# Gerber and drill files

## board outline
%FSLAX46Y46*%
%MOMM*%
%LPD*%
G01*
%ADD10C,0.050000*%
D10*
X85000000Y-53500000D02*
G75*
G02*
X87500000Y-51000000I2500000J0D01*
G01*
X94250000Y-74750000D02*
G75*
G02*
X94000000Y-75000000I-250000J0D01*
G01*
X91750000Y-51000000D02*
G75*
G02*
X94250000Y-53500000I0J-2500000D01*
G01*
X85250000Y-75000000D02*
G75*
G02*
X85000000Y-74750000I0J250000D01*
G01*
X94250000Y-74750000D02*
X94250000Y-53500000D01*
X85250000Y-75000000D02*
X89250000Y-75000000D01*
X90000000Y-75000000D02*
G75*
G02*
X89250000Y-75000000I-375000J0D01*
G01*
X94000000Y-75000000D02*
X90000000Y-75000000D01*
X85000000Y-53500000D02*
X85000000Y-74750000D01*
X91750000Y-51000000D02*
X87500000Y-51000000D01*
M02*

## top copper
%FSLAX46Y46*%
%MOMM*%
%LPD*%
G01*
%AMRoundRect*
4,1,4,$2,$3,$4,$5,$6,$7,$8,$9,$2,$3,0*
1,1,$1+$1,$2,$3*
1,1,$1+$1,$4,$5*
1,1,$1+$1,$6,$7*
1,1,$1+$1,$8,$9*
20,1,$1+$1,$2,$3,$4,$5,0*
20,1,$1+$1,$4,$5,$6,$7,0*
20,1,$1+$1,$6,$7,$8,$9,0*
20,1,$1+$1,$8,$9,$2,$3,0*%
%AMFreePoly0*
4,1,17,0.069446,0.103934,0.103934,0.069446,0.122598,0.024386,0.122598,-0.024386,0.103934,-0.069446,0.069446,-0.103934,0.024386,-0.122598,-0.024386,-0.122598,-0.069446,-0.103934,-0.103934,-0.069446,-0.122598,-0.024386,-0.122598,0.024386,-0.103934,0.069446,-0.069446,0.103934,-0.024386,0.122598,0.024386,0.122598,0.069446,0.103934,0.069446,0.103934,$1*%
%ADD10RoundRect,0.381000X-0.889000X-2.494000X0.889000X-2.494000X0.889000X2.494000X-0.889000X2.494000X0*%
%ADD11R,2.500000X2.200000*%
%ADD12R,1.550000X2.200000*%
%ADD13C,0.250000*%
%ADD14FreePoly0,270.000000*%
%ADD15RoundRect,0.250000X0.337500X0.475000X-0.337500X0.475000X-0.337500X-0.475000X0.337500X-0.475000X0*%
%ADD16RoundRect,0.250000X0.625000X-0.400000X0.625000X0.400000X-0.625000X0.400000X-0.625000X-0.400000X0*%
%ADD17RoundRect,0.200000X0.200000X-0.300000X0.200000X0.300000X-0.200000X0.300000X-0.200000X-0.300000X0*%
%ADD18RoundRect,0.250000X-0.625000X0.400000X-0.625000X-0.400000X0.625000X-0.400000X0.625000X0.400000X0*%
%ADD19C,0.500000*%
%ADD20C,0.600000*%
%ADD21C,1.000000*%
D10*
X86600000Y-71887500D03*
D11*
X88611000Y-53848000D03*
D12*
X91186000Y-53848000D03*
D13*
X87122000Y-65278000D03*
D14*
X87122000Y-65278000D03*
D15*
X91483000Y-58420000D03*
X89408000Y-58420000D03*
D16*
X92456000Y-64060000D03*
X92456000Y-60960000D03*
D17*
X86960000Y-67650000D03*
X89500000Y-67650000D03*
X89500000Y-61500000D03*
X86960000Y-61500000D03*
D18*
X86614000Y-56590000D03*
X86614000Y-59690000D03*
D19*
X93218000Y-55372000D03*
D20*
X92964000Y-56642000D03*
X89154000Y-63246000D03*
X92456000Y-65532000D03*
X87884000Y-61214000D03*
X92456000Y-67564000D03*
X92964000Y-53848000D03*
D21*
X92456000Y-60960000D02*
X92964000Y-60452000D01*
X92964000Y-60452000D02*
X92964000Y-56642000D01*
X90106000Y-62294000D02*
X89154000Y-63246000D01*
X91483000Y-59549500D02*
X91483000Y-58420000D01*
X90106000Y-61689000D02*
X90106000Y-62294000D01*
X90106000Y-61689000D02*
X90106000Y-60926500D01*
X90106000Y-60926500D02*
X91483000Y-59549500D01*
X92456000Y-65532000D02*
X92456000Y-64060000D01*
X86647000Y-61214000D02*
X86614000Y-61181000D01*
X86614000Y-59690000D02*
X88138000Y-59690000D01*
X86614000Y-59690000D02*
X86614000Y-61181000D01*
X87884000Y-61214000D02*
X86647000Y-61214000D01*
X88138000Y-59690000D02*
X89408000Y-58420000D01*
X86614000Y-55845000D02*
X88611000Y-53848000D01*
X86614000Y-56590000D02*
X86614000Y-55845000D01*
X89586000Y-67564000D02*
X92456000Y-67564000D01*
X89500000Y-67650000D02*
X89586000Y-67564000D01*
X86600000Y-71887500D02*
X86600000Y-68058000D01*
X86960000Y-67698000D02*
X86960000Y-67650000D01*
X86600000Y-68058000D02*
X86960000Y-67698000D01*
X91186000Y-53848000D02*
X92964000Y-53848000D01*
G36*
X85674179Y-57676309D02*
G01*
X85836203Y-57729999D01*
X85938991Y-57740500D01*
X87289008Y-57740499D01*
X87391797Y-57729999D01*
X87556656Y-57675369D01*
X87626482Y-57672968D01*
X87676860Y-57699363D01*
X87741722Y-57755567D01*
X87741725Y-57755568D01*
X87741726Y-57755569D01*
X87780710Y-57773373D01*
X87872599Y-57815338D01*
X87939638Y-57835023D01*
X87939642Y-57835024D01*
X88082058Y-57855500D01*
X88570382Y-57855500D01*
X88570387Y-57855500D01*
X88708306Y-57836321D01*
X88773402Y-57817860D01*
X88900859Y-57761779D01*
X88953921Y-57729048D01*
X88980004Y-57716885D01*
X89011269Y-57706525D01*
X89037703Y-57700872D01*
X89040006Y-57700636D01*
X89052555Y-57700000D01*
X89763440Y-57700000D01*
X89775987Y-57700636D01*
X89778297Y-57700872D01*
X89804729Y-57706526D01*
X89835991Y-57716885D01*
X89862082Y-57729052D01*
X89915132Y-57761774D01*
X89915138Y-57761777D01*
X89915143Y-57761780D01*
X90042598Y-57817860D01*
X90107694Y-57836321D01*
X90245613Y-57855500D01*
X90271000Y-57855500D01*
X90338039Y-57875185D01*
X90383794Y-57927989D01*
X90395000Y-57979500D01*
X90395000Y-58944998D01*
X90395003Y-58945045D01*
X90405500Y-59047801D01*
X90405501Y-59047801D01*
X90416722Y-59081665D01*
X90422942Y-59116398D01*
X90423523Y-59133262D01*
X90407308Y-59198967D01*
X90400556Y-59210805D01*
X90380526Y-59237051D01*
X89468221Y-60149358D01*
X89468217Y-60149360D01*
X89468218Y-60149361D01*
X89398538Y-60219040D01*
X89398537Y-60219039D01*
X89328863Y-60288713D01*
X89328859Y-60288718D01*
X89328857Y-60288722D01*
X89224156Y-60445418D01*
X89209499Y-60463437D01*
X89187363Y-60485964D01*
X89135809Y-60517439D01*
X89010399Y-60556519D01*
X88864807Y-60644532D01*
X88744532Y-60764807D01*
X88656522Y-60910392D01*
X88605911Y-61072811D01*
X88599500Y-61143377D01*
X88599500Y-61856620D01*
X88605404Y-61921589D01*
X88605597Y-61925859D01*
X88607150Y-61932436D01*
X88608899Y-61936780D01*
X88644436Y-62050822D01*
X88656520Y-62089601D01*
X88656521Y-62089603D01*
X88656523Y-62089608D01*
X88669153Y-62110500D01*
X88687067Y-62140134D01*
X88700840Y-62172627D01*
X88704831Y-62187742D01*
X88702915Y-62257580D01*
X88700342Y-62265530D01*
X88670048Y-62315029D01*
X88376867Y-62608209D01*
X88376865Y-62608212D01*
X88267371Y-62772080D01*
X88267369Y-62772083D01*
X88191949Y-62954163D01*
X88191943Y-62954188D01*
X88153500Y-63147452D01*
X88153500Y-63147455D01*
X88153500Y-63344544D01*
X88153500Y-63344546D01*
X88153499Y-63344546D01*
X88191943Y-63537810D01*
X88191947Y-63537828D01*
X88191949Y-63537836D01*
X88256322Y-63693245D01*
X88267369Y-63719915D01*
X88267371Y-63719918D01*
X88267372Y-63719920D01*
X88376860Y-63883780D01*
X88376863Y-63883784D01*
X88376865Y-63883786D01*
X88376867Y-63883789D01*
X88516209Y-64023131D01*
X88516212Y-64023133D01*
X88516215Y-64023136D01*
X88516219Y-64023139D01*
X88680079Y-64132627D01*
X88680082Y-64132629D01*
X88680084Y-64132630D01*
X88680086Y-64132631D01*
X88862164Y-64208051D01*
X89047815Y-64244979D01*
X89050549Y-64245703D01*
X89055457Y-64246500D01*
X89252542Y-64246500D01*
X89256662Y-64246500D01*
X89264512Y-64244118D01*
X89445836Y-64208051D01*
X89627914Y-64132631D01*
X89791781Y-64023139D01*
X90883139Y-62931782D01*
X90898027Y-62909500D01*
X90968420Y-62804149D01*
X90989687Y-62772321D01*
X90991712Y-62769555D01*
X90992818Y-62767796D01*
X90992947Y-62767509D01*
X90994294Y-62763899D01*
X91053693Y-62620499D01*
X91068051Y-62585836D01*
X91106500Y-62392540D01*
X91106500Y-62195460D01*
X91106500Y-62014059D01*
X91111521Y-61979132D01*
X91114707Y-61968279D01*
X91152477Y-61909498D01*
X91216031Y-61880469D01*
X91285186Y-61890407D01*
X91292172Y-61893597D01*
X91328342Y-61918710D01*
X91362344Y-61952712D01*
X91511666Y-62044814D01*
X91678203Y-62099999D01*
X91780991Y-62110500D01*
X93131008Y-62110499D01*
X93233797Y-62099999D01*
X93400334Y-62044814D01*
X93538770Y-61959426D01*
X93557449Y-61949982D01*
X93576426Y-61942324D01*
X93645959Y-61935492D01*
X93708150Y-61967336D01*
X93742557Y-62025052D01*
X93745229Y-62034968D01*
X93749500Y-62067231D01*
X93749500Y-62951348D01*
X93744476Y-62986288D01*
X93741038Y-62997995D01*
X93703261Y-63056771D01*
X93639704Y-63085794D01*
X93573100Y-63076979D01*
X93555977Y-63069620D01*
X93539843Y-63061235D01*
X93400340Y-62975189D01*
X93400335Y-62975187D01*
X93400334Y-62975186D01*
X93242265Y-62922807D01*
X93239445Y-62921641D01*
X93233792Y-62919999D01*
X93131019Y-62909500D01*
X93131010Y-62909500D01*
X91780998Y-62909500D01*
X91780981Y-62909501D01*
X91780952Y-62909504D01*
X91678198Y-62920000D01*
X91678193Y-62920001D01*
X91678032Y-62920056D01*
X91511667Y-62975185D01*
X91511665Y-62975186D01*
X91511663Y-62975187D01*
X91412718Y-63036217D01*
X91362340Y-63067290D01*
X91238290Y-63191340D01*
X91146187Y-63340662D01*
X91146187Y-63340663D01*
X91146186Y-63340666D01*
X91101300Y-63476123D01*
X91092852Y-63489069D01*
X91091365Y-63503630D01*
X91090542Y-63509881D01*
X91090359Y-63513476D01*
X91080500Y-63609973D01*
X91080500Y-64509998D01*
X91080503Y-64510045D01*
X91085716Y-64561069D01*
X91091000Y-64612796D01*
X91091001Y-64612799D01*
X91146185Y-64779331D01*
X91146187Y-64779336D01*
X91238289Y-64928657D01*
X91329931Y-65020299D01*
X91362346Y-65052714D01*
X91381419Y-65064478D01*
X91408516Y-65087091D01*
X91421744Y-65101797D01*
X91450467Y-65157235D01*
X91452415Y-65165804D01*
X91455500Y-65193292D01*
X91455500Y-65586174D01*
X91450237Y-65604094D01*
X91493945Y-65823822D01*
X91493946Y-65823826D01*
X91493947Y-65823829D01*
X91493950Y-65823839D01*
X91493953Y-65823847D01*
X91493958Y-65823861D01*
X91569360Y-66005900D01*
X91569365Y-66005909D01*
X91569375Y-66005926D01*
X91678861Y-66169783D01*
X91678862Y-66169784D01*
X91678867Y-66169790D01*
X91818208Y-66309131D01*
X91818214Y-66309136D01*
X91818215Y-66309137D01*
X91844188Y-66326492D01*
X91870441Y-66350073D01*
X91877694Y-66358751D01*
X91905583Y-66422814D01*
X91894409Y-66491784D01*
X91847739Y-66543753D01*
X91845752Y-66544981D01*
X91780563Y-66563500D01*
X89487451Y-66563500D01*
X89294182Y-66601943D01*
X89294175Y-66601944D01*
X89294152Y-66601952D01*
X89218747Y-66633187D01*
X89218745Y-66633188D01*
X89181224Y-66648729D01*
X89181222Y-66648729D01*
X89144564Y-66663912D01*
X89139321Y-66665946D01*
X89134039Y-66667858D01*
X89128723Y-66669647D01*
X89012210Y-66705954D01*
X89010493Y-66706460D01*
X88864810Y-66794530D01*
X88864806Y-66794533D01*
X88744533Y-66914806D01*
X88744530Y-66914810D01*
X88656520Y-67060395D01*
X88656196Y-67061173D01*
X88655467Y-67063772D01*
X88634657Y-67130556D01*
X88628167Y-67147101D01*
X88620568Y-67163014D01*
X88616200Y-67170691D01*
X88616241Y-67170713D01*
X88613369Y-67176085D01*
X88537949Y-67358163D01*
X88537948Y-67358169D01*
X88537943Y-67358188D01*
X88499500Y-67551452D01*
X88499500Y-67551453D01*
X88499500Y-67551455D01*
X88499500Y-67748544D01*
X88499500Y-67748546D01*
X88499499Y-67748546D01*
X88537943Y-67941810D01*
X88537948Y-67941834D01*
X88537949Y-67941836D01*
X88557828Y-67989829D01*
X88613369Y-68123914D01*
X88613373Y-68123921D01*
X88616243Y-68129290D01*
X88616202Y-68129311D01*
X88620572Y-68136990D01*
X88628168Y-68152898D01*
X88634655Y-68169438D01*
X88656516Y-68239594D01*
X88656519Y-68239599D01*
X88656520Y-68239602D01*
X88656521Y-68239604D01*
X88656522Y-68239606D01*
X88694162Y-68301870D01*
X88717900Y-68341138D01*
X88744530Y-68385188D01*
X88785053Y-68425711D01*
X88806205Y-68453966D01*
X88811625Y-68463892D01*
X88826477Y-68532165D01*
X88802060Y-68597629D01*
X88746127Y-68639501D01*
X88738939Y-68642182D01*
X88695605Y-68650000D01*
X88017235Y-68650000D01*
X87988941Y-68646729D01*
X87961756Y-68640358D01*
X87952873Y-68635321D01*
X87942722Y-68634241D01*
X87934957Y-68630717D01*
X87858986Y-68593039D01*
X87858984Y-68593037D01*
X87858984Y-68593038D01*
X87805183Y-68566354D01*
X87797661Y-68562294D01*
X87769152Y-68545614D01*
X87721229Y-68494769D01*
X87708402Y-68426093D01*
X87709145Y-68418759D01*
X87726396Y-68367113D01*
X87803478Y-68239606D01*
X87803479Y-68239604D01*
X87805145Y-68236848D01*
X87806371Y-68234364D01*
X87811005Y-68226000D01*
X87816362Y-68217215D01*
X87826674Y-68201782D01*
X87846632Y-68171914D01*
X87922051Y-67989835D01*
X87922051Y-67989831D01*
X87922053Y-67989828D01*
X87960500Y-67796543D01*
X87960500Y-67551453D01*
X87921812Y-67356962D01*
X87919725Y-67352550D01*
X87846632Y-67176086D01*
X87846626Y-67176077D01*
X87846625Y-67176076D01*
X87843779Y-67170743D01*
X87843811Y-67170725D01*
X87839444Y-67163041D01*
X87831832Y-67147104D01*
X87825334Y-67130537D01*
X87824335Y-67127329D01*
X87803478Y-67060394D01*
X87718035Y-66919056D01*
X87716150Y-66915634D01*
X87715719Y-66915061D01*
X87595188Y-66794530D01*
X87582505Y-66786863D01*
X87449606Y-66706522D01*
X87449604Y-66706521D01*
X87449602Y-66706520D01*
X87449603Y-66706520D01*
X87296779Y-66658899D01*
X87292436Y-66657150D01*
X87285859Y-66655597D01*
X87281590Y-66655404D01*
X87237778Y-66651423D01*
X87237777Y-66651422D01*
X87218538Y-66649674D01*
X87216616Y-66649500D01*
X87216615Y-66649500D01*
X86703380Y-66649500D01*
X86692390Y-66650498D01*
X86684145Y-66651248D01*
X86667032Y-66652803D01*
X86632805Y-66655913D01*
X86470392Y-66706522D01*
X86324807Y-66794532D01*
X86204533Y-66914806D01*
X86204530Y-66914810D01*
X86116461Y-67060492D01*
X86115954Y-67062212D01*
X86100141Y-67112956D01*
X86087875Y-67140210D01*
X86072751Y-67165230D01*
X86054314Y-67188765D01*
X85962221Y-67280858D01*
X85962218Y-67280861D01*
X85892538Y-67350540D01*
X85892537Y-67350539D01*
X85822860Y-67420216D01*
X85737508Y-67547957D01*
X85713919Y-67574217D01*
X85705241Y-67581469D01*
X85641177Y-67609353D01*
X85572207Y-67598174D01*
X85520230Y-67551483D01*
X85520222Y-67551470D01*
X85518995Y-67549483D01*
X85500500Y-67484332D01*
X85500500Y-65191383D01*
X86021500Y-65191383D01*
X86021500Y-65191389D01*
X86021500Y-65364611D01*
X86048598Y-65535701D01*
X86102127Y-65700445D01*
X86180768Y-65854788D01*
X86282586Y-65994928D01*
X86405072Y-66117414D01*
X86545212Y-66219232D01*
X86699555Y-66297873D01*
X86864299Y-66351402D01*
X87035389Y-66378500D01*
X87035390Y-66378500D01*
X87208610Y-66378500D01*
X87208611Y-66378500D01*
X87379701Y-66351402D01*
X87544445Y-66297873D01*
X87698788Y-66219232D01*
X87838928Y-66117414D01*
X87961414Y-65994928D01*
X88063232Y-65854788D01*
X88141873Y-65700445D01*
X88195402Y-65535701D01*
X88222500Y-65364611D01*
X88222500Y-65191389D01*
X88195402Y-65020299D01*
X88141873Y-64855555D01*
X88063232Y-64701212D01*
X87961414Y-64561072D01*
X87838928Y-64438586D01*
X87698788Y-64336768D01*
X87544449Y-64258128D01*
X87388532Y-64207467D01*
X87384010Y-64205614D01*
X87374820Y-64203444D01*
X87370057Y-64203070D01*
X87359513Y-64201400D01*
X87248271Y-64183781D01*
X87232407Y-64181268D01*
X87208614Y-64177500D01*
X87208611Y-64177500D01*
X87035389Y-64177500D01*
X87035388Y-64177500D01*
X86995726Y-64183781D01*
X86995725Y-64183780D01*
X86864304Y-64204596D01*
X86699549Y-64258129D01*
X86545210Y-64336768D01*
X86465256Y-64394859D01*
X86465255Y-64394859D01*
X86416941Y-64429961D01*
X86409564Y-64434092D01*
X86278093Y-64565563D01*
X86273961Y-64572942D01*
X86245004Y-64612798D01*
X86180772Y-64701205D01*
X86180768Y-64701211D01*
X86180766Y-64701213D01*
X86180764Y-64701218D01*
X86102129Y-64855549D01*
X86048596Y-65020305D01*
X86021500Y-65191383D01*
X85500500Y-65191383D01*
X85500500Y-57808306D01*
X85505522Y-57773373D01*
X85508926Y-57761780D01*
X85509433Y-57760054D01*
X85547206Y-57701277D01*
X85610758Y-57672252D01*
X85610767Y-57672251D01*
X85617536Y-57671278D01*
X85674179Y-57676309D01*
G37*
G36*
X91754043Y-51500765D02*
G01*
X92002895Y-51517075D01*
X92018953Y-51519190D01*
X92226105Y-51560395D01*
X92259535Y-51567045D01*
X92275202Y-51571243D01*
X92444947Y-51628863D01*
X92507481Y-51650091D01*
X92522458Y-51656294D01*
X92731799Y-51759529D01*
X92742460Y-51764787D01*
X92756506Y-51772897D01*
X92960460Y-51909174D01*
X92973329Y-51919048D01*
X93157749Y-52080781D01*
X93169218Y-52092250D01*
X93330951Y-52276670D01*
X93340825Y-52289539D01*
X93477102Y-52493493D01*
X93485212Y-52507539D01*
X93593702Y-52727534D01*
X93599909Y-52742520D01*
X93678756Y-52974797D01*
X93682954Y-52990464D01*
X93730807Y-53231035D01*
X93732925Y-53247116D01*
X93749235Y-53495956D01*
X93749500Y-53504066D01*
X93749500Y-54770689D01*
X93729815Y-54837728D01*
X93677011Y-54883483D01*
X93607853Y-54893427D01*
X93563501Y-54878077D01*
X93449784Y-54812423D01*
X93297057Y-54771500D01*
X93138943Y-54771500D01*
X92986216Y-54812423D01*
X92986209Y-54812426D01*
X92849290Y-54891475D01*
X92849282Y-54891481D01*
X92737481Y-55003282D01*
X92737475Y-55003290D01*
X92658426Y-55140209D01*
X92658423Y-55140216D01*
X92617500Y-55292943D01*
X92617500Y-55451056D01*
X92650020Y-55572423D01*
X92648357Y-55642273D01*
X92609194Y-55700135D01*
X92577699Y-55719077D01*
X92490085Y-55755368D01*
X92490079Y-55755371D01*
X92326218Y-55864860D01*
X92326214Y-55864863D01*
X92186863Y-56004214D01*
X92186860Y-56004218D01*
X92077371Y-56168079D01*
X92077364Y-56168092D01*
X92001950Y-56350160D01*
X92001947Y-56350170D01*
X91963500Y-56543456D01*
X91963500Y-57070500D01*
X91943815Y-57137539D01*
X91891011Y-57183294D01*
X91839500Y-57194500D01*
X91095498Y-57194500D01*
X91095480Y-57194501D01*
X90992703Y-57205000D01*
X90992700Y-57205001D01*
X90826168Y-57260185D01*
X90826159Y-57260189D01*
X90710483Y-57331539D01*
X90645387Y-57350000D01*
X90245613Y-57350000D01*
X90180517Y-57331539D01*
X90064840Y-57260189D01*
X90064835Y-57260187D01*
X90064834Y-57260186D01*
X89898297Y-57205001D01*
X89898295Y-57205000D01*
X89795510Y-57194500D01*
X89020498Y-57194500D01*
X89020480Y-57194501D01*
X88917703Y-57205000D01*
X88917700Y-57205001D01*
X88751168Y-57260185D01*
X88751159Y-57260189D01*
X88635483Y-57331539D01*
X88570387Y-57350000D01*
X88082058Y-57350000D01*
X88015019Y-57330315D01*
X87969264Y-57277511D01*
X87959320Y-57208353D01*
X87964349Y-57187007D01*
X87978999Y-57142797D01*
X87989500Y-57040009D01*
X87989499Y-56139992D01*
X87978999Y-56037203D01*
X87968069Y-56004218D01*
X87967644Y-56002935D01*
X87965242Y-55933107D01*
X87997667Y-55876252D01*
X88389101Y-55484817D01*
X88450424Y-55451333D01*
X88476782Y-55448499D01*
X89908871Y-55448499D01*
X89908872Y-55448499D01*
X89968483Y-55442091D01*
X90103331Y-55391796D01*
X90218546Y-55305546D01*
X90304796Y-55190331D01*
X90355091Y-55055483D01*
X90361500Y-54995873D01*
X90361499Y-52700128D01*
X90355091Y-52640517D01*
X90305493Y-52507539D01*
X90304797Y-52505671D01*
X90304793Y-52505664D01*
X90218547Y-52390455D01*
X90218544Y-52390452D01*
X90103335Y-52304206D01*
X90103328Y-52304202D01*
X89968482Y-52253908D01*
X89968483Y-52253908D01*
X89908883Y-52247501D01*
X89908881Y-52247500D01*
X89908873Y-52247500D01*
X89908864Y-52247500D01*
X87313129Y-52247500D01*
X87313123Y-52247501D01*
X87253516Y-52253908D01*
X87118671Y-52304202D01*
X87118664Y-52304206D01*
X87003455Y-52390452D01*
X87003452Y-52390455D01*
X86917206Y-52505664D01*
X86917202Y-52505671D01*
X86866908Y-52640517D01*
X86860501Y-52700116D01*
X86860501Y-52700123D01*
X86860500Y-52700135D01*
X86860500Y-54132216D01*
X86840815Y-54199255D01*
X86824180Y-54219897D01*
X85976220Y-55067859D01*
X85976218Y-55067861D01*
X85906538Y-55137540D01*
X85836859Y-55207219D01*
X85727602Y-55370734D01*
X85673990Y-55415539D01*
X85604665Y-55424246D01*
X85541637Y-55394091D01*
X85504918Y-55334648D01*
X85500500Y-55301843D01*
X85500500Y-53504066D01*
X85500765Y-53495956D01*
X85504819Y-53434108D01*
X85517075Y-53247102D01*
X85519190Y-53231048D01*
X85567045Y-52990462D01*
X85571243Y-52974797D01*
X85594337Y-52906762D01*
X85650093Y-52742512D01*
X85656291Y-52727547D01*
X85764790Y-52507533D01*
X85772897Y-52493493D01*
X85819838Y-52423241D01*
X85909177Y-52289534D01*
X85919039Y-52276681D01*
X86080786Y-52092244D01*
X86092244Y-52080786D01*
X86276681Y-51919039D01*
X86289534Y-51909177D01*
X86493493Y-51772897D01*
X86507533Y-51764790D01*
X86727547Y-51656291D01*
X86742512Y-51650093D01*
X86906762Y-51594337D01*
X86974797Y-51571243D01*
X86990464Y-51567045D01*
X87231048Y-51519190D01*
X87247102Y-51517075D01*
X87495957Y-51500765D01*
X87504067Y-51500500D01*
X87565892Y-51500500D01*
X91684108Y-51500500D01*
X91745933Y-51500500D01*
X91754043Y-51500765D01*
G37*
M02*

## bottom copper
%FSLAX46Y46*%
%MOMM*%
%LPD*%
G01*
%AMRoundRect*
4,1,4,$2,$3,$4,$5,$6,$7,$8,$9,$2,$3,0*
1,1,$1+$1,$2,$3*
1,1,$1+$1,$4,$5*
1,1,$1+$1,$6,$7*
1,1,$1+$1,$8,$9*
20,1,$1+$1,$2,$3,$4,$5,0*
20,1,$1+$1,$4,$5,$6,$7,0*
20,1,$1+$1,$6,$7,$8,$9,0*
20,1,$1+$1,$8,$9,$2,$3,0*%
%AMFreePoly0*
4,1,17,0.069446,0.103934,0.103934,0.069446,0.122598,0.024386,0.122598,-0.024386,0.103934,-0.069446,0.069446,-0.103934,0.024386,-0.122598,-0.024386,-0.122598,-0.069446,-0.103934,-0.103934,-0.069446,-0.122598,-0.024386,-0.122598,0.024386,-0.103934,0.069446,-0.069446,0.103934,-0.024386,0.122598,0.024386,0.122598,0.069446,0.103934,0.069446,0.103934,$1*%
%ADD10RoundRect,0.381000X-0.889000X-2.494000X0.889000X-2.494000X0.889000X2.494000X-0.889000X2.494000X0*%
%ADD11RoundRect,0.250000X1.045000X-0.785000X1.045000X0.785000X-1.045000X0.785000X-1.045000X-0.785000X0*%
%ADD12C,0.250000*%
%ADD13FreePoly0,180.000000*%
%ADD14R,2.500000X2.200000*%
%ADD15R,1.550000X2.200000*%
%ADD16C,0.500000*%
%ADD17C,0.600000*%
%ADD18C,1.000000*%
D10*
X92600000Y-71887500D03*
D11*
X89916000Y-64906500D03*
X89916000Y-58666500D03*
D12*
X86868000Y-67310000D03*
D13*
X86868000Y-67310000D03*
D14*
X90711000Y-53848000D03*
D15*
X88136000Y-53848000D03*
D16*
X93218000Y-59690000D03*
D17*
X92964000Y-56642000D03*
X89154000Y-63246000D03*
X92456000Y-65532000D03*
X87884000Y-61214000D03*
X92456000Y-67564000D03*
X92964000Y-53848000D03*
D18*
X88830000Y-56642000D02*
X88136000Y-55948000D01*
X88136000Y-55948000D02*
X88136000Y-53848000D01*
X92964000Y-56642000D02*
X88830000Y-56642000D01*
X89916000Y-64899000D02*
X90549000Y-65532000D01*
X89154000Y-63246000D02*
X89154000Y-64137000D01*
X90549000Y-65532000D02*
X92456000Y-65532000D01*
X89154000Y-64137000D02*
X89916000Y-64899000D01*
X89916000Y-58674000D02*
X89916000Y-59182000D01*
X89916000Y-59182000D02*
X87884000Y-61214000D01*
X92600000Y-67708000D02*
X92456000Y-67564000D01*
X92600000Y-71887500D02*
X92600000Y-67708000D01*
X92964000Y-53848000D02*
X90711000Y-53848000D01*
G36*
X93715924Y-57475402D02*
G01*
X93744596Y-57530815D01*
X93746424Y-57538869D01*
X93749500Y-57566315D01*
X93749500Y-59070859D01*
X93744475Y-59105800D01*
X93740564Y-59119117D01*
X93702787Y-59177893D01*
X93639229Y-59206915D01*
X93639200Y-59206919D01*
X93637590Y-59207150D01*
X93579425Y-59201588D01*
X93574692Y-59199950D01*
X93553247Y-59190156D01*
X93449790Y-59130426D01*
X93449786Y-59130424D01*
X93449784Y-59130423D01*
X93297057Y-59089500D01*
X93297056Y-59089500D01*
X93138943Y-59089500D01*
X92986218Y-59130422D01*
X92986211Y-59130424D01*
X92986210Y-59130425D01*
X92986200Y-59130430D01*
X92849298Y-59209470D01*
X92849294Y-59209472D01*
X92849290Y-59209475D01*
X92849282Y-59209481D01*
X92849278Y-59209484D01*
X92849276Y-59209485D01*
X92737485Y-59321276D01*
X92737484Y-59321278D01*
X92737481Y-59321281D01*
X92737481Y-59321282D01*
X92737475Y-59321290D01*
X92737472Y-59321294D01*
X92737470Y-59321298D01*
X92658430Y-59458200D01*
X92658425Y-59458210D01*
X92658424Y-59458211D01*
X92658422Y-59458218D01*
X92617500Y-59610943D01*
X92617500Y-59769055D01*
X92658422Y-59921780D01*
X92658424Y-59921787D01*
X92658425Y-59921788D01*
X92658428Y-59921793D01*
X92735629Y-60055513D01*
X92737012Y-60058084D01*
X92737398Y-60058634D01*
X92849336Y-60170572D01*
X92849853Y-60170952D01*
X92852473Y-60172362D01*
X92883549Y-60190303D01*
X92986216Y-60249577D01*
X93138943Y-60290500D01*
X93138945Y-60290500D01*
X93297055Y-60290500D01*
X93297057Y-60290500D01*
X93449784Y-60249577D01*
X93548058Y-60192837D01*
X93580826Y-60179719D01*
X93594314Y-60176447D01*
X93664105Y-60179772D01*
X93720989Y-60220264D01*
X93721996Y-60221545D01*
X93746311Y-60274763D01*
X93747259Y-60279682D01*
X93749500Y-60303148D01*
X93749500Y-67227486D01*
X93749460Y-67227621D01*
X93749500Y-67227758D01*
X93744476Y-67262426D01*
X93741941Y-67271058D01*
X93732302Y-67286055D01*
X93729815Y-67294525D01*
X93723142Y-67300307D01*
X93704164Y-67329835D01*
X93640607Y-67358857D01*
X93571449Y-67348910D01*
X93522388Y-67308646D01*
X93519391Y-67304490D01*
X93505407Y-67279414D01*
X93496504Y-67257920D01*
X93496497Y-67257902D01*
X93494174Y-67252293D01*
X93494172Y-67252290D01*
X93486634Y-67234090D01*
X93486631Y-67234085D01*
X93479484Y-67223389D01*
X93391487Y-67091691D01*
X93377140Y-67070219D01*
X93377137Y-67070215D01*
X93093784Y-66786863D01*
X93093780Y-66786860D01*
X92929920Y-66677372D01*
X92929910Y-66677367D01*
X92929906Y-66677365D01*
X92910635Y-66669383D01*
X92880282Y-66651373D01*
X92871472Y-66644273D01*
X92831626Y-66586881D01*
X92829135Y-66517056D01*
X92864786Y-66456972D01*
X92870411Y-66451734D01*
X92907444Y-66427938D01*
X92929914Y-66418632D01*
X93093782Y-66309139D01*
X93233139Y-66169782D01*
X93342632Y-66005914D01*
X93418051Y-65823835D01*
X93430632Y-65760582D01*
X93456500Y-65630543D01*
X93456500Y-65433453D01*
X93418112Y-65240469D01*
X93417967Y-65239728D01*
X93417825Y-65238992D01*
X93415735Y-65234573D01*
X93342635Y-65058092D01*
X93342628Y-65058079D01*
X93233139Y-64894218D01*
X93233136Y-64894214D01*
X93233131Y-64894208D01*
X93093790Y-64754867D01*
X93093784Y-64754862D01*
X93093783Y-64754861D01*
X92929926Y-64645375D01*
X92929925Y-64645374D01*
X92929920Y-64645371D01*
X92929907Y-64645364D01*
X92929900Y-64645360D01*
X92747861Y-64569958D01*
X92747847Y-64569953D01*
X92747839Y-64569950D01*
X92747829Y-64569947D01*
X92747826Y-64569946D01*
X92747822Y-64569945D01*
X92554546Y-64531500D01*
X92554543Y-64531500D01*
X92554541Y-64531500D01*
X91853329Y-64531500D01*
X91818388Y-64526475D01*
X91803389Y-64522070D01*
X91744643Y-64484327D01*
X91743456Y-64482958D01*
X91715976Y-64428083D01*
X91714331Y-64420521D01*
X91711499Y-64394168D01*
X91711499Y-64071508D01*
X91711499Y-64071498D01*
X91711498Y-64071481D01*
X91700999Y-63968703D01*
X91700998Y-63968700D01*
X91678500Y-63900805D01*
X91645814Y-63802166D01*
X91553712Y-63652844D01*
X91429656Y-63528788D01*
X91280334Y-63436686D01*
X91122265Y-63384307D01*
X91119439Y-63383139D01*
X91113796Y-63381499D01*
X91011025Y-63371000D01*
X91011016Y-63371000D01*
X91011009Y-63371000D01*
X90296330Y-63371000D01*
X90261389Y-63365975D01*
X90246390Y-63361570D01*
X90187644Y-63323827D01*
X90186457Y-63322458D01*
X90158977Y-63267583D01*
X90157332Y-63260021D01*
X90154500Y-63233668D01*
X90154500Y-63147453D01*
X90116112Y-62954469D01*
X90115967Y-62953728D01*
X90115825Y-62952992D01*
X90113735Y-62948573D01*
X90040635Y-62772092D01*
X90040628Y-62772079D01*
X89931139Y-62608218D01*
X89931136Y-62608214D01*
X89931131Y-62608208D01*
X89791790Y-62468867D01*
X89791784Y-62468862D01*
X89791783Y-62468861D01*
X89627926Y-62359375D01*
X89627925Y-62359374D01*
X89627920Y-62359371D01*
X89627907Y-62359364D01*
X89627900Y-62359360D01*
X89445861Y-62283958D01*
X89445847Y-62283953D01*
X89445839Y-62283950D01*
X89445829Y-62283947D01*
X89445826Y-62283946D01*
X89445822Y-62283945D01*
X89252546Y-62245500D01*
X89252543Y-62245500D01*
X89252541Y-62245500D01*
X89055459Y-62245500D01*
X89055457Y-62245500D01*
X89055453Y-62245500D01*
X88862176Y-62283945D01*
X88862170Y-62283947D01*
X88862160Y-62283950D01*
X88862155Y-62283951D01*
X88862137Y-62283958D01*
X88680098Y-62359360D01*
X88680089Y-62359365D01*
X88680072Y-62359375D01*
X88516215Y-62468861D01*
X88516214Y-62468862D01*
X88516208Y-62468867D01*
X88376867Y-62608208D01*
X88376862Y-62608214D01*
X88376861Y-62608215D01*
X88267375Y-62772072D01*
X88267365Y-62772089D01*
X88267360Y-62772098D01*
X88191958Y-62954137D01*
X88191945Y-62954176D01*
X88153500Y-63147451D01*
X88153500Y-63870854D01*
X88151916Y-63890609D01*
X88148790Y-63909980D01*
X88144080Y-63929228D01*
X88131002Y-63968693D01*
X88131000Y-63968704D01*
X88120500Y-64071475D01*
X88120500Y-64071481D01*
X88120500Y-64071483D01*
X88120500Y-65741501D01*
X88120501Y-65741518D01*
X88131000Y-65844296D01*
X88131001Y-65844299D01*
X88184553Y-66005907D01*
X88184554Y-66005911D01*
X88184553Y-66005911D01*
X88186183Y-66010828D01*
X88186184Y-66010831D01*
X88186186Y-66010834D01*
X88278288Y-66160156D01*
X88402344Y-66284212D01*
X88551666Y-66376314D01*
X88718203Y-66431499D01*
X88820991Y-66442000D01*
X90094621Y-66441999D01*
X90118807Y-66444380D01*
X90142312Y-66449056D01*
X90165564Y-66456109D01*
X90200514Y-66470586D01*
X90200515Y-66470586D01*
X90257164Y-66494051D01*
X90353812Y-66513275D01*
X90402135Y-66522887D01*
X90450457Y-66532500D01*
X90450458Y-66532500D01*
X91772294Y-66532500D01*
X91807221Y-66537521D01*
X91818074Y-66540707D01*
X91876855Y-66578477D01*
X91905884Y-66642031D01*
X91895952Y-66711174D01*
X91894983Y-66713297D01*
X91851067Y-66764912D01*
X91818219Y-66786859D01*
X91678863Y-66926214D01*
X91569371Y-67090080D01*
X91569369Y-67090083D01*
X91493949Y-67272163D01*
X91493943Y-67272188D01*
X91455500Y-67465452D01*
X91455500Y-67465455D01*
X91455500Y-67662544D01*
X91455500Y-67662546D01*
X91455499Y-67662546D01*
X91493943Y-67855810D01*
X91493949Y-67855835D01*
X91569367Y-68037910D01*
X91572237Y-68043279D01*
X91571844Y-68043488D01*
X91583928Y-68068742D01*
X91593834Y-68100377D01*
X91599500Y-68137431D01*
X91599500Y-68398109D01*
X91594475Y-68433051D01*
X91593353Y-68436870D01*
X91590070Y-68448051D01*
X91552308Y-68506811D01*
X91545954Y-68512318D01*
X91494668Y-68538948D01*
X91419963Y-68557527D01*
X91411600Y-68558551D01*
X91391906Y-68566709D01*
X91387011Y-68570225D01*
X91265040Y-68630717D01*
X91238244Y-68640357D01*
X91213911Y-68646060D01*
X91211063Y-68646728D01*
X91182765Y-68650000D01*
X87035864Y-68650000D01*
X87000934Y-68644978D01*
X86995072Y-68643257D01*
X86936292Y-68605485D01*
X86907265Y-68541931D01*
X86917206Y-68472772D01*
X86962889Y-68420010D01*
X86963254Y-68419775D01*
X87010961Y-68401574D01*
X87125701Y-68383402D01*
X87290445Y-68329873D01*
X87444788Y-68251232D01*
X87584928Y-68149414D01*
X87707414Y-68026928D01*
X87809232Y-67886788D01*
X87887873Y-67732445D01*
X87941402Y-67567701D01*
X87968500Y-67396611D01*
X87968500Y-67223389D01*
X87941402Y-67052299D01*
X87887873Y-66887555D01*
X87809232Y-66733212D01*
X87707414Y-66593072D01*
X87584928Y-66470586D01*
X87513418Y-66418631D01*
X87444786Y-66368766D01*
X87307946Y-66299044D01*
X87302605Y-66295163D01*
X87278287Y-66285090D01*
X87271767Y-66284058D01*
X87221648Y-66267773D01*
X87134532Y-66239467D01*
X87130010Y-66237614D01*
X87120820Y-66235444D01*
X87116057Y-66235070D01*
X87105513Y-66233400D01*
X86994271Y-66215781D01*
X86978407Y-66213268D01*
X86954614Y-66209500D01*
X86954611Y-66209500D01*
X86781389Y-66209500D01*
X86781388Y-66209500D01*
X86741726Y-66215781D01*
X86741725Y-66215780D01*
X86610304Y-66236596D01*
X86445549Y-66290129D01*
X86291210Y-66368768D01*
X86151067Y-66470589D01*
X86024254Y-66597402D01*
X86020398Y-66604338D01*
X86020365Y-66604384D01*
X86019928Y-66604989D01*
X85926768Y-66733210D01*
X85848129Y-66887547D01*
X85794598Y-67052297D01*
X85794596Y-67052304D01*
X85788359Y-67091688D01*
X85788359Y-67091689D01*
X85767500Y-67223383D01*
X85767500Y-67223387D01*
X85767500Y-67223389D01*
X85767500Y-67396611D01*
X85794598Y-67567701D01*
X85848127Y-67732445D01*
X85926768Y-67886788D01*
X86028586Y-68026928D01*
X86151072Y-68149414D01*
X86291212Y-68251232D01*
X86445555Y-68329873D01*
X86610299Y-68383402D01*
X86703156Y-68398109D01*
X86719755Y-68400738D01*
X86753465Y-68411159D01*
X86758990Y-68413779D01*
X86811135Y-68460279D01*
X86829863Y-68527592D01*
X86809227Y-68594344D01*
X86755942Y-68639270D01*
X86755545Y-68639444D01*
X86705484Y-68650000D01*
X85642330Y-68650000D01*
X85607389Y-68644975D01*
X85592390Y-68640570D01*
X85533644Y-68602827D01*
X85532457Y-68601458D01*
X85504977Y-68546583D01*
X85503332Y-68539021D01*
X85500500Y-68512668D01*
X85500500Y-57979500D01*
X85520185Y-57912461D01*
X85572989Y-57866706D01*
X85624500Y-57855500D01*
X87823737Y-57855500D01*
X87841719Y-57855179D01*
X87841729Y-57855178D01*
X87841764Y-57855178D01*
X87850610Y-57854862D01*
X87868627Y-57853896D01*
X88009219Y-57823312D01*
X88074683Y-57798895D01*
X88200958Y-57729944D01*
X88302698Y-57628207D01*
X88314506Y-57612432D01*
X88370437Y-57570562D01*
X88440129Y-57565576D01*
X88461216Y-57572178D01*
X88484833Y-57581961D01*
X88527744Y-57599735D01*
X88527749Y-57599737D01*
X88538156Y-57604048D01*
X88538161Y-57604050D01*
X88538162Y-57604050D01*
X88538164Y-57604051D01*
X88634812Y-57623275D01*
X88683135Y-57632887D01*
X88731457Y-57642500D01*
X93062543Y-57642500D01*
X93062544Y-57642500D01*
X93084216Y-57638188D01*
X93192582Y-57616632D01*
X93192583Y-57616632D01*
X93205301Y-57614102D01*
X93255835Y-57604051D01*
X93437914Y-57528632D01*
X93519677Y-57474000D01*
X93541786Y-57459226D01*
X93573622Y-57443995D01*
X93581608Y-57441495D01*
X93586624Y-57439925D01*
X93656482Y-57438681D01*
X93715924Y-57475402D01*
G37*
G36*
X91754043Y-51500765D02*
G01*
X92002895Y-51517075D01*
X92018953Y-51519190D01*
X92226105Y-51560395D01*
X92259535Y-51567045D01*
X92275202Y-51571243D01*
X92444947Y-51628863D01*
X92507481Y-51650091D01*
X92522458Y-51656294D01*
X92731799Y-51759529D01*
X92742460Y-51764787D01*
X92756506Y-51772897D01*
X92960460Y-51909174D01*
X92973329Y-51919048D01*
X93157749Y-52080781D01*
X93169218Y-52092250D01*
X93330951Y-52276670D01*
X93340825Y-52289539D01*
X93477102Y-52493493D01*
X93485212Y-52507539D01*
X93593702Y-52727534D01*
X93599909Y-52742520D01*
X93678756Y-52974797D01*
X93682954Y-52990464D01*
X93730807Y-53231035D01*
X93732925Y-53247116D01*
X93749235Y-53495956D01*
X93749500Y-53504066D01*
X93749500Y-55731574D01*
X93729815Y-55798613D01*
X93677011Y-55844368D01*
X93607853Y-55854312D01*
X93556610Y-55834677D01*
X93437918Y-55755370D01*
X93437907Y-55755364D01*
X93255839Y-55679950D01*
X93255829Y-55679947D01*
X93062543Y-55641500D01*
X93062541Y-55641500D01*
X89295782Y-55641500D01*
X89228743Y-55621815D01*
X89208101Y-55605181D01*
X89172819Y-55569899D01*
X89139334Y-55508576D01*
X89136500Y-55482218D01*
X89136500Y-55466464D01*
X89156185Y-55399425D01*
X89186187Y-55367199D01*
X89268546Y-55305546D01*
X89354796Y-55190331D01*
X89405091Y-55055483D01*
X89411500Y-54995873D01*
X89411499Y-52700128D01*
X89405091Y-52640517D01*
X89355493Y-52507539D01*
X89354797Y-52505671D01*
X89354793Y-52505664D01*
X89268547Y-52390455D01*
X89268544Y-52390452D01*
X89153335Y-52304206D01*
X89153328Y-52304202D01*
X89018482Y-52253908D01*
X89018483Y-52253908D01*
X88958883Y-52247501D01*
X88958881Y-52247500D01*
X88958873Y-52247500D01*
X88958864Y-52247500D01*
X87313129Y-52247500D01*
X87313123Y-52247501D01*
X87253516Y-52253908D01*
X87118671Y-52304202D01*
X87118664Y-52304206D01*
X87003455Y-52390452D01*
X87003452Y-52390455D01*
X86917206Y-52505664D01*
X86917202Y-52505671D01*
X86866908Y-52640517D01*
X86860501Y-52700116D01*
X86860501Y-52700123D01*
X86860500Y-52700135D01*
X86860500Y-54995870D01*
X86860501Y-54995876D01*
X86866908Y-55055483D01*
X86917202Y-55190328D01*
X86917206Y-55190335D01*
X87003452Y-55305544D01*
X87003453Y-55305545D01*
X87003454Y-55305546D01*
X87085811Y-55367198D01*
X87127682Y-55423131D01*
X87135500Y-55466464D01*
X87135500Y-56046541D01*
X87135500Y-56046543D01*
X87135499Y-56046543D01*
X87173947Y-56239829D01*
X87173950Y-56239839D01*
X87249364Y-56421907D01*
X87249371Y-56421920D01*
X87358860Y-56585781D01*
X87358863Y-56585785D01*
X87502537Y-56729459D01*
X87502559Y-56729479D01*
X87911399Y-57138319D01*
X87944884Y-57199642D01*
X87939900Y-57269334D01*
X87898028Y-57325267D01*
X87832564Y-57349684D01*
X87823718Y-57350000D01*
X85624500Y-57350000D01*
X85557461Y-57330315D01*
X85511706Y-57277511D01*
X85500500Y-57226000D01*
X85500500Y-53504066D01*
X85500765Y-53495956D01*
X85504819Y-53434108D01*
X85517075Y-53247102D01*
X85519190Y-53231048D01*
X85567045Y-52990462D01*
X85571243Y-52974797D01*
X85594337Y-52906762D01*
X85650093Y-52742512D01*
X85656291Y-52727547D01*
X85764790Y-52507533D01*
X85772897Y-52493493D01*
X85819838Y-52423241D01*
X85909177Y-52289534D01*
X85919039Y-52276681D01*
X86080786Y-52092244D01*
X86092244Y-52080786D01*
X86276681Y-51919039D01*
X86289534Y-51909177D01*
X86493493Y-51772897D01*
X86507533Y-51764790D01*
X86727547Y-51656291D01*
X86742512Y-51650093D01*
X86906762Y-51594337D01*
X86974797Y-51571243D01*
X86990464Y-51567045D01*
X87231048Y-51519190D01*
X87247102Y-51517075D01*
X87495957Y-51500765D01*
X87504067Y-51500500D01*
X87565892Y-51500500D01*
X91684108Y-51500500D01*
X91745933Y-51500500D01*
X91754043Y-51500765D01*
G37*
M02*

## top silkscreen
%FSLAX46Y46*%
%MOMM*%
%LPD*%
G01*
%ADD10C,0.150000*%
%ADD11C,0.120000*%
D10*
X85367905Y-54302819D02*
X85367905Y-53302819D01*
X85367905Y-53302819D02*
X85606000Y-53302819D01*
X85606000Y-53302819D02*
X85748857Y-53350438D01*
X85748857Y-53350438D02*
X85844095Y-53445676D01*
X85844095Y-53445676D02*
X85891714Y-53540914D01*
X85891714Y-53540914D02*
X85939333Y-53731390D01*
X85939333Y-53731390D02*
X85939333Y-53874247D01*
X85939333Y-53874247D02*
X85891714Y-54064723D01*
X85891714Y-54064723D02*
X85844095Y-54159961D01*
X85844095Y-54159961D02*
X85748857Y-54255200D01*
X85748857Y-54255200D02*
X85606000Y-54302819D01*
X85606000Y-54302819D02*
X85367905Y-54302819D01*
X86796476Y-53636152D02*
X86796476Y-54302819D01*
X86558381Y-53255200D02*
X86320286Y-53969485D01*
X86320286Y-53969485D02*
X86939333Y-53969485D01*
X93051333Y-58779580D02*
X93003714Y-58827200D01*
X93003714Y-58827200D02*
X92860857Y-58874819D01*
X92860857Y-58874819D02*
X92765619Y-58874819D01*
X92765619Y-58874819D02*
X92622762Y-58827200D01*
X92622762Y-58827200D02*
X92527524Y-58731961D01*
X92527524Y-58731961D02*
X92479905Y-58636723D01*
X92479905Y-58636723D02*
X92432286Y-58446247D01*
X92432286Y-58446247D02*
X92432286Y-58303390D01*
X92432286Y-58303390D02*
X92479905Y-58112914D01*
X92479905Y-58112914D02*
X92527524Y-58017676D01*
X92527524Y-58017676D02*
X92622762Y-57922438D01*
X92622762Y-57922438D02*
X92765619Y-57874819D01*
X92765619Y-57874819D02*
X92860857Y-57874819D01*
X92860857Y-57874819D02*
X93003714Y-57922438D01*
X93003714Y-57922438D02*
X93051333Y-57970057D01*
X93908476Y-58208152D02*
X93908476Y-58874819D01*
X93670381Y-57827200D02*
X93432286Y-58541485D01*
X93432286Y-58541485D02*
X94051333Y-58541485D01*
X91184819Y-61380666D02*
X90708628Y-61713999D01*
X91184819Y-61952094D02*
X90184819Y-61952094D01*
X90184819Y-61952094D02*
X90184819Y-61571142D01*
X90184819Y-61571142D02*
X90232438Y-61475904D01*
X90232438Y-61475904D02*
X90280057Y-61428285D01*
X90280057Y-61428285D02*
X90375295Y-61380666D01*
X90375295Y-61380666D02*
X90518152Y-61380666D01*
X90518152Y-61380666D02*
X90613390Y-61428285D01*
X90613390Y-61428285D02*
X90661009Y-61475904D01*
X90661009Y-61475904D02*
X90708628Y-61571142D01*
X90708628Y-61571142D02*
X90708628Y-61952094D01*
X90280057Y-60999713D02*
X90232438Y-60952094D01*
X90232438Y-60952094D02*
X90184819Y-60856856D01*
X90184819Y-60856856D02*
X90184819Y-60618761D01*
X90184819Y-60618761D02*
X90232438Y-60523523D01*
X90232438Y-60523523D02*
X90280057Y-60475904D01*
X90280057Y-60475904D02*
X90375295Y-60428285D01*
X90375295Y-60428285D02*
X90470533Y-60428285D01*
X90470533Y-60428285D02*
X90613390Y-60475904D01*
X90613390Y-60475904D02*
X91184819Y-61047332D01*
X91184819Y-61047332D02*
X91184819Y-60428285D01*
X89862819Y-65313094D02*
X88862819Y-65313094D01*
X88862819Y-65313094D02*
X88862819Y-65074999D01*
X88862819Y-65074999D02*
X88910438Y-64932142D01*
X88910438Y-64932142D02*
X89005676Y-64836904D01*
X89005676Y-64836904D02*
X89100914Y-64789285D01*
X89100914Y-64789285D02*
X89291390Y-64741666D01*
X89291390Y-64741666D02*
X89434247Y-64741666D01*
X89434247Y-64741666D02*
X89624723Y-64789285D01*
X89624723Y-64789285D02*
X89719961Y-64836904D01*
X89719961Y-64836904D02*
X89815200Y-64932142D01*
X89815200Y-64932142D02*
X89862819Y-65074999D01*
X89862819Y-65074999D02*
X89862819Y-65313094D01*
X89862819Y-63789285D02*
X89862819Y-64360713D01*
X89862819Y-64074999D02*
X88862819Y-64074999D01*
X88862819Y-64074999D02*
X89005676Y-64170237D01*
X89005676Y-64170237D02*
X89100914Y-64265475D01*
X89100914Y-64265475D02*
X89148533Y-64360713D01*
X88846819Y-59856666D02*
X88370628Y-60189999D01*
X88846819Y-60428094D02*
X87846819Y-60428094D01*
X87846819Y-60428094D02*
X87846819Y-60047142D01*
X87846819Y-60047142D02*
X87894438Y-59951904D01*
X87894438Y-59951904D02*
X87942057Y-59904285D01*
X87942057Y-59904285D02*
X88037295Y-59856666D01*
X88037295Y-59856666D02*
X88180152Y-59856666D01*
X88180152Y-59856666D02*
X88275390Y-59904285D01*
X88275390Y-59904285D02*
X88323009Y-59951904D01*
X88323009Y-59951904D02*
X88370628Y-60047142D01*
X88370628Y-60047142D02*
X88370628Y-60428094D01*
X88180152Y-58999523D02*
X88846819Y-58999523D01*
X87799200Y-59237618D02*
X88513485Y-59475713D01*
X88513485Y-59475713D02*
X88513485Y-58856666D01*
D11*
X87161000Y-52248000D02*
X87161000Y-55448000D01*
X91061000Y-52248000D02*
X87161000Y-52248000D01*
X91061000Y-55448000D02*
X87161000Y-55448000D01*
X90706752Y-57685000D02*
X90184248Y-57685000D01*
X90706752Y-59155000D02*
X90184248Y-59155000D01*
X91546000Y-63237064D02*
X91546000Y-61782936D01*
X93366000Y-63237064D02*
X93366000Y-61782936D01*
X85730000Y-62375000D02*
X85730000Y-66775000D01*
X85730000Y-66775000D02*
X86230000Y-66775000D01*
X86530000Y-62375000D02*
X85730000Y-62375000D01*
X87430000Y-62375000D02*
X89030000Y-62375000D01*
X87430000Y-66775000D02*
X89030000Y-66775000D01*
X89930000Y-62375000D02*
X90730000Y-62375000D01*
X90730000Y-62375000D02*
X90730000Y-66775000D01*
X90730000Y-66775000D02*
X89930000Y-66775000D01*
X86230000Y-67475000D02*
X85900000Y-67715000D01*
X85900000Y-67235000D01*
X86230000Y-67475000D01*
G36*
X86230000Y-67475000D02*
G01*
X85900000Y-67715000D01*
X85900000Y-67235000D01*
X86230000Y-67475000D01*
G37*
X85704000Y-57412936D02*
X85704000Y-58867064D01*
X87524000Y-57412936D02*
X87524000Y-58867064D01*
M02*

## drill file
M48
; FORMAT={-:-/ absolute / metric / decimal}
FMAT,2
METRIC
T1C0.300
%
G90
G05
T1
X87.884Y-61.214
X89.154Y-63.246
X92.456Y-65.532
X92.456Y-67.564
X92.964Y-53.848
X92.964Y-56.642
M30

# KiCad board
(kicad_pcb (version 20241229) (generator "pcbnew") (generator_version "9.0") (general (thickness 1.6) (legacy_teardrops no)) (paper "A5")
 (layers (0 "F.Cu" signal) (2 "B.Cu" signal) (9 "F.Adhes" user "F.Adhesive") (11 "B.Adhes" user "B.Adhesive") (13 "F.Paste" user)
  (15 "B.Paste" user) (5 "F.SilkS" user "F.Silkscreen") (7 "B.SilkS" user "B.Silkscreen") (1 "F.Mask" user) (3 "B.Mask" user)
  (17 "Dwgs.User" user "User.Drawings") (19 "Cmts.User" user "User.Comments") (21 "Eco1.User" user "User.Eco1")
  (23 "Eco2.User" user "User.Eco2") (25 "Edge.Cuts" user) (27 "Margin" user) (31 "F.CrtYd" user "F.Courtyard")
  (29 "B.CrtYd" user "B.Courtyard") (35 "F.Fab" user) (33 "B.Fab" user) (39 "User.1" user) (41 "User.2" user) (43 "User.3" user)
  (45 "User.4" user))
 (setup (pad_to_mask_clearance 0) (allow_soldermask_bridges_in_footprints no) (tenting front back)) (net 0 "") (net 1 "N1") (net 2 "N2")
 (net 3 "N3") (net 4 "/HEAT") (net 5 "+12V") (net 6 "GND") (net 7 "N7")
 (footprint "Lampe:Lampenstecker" (layer "F.Cu") (at 89.6 68.3875)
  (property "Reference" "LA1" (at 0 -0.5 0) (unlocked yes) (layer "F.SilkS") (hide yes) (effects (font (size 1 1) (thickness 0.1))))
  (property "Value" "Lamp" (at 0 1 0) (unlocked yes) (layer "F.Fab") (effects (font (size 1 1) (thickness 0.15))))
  (pad "1" smd roundrect (at -3 3.5) (size 2.54 5.75) (layers "F.Cu" "F.Mask" "F.Paste") (roundrect_rratio 0.15) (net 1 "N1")
   (thermal_bridge_angle 45))
  (pad "2" smd roundrect (at 3 3.5) (size 2.54 5.75) (layers "B.Cu" "B.Mask" "B.Paste") (roundrect_rratio 0.15) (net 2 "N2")
   (thermal_bridge_angle 45)))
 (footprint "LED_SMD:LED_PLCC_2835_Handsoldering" (layer "F.Cu") (at 89.661 53.848)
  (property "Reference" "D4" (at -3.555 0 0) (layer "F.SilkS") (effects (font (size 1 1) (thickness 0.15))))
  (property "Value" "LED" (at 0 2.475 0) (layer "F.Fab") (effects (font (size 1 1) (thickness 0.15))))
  (fp_line (start -2.5 -1.6) (end -2.5 1.6) (stroke (width 0.12) (type solid)) (layer "F.SilkS"))
  (fp_line (start 1.4 -1.6) (end -2.5 -1.6) (stroke (width 0.12) (type solid)) (layer "F.SilkS"))
  (fp_line (start 1.4 1.6) (end -2.5 1.6) (stroke (width 0.12) (type solid)) (layer "F.SilkS"))
  (pad "1" smd rect (at -1.05 0) (size 2.5 2.2) (layers "F.Cu" "F.Mask" "F.Paste") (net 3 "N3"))
  (pad "2" smd rect (at 1.525 0) (size 1.55 2.2) (layers "F.Cu" "F.Mask" "F.Paste") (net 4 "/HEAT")))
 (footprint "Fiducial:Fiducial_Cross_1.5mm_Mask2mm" (layer "F.Cu") (at 87.122 65.278 -90)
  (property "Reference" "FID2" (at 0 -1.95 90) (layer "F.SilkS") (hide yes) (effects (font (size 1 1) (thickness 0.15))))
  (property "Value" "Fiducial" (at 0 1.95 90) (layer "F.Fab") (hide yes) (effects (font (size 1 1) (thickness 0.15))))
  (pad "" smd circle (at 0 0 270) (size 0.25 0.25) (layers "F.Cu" "F.Mask") (solder_mask_margin 0.875) (clearance 0.975))
  (pad "" smd custom (at 0 0 270) (size 0.25 0.25) (layers "F.Cu" "F.Mask") (options (clearance outline) (anchor circle)) (primitives)))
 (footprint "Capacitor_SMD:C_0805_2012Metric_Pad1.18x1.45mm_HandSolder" (layer "F.Cu") (at 90.4455 58.42 180)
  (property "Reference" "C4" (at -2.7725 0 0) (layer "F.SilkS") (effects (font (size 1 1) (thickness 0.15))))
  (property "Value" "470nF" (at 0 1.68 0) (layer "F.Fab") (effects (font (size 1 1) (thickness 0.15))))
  (fp_line (start -0.261252 0.735) (end 0.261252 0.735) (stroke (width 0.12) (type solid)) (layer "F.SilkS"))
  (fp_line (start -0.261252 -0.735) (end 0.261252 -0.735) (stroke (width 0.12) (type solid)) (layer "F.SilkS"))
  (pad "1" smd roundrect (at -1.0375 0 180) (size 1.175 1.45) (layers "F.Cu" "F.Mask" "F.Paste") (roundrect_rratio 0.212766) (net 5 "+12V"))
  (pad "2" smd roundrect (at 1.0375 0 180) (size 1.175 1.45) (layers "F.Cu" "F.Mask" "F.Paste") (roundrect_rratio 0.212766) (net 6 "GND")))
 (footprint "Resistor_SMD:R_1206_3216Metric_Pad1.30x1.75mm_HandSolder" (layer "F.Cu") (at 92.456 62.51 90)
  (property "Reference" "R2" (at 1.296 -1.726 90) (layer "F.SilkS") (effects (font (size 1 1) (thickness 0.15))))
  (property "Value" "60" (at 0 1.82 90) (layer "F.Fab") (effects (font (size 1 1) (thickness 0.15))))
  (fp_line (start -0.727064 -0.91) (end 0.727064 -0.91) (stroke (width 0.12) (type solid)) (layer "F.SilkS"))
  (fp_line (start -0.727064 0.91) (end 0.727064 0.91) (stroke (width 0.12) (type solid)) (layer "F.SilkS"))
  (pad "1" smd roundrect (at -1.55 0 90) (size 1.3 1.75) (layers "F.Cu" "F.Mask" "F.Paste") (roundrect_rratio 0.192308) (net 5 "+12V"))
  (pad "2" smd roundrect (at 1.55 0 90) (size 1.3 1.75) (layers "F.Cu" "F.Mask" "F.Paste") (roundrect_rratio 0.192308) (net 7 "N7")))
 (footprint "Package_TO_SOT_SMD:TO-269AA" (layer "F.Cu") (at 88.23 64.575 90)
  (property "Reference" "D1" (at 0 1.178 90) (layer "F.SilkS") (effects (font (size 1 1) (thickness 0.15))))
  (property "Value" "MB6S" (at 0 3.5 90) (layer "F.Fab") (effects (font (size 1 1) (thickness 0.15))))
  (fp_line (start 2.2 -2.5) (end -2.2 -2.5) (stroke (width 0.12) (type solid)) (layer "F.SilkS"))
  (fp_line (start -2.2 -2.5) (end -2.2 -2) (stroke (width 0.12) (type solid)) (layer "F.SilkS"))
  (fp_line (start 2.2 -1.7) (end 2.2 -2.5) (stroke (width 0.12) (type solid)) (layer "F.SilkS"))
  (fp_line (start 2.2 -0.8) (end 2.2 0.8) (stroke (width 0.12) (type solid)) (layer "F.SilkS"))
  (fp_line (start -2.2 -0.8) (end -2.2 0.8) (stroke (width 0.12) (type solid)) (layer "F.SilkS"))
  (fp_line (start 2.2 1.7) (end 2.2 2.5) (stroke (width 0.12) (type solid)) (layer "F.SilkS"))
  (fp_line (start 2.2 2.5) (end -2.2 2.5) (stroke (width 0.12) (type solid)) (layer "F.SilkS"))
  (fp_line (start -2.2 2.5) (end -2.2 1.7) (stroke (width 0.12) (type solid)) (layer "F.SilkS"))
  (fp_poly
   (pts (xy -2.9 -2) (xy -3.14 -2.33) (xy -2.66 -2.33) (xy -2.9 -2)) (stroke (width 0.12) (type solid)) (fill yes) (layer "F.SilkS"))
  (pad "1" smd roundrect (at -3.075 -1.27 90) (size 1 0.8) (layers "F.Cu" "F.Mask" "F.Paste") (roundrect_rratio 0.25) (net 1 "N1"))
  (pad "2" smd roundrect (at -3.075 1.27 90) (size 1 0.8) (layers "F.Cu" "F.Mask" "F.Paste") (roundrect_rratio 0.25) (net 2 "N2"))
  (pad "3" smd roundrect (at 3.075 1.27 90) (size 1 0.8) (layers "F.Cu" "F.Mask" "F.Paste") (roundrect_rratio 0.25) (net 5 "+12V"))
  (pad "4" smd roundrect (at 3.075 -1.27 90) (size 1 0.8) (layers "F.Cu" "F.Mask" "F.Paste") (roundrect_rratio 0.25) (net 6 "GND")))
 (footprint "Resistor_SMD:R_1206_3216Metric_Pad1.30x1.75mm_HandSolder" (layer "F.Cu") (at 86.614 58.14 -90)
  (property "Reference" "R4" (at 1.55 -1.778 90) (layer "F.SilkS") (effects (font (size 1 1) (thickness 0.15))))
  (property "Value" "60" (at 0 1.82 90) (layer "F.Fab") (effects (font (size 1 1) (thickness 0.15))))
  (fp_line (start -0.727064 0.91) (end 0.727064 0.91) (stroke (width 0.12) (type solid)) (layer "F.SilkS"))
  (fp_line (start -0.727064 -0.91) (end 0.727064 -0.91) (stroke (width 0.12) (type solid)) (layer "F.SilkS"))
  (pad "1" smd roundrect (at -1.55 0 270) (size 1.3 1.75) (layers "F.Cu" "F.Mask" "F.Paste") (roundrect_rratio 0.192308) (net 3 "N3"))
  (pad "2" smd roundrect (at 1.55 0 270) (size 1.3 1.75) (layers "F.Cu" "F.Mask" "F.Paste") (roundrect_rratio 0.192308) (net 6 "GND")))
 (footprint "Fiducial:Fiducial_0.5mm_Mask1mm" (layer "F.Cu") (at 93.218 55.372)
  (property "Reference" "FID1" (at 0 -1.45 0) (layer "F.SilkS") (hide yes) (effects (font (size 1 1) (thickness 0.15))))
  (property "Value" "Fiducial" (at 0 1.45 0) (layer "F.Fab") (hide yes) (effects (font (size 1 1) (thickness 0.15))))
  (pad "" smd circle (at 0 0) (size 0.5 0.5) (layers "F.Cu" "F.Mask") (solder_mask_margin 0.25) (clearance 0.35)))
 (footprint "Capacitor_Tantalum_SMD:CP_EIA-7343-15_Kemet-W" (layer "B.Cu") (at 89.916 61.7865 90)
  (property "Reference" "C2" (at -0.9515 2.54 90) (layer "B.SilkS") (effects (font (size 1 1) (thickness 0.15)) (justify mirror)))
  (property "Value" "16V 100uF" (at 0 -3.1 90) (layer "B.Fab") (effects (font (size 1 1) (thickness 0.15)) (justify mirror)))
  (pad "1" smd roundrect (at -3.12 0 90) (size 2.07 2.59) (layers "B.Cu" "B.Mask" "B.Paste") (roundrect_rratio 0.120773) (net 5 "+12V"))
  (pad "2" smd roundrect (at 3.12 0 90) (size 2.07 2.59) (layers "B.Cu" "B.Mask" "B.Paste") (roundrect_rratio 0.120773) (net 6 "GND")))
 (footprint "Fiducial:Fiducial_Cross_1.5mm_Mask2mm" (layer "B.Cu") (at 86.868 67.31 180)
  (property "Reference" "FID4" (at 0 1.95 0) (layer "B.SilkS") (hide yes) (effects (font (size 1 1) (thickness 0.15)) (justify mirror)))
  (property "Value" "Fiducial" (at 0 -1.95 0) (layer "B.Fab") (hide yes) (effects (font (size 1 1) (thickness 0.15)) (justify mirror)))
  (pad "" smd circle (at 0 0 180) (size 0.25 0.25) (layers "B.Cu" "B.Mask") (solder_mask_margin 0.875) (clearance 0.975))
  (pad "" smd custom (at 0 0 180) (size 0.25 0.25) (layers "B.Cu" "B.Mask") (options (clearance outline) (anchor circle)) (primitives)))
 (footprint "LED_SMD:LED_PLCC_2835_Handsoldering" (layer "B.Cu") (at 89.661 53.848 180)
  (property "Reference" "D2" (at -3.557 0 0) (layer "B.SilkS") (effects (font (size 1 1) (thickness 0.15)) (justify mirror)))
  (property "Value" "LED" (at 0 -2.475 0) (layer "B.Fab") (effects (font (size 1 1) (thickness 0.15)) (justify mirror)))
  (pad "1" smd rect (at -1.05 0 180) (size 2.5 2.2) (layers "B.Cu" "B.Mask" "B.Paste") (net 4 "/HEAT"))
  (pad "2" smd rect (at 1.525 0 180) (size 1.55 2.2) (layers "B.Cu" "B.Mask" "B.Paste") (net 7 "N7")))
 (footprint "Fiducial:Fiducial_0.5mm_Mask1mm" (layer "B.Cu") (at 93.218 59.69 180)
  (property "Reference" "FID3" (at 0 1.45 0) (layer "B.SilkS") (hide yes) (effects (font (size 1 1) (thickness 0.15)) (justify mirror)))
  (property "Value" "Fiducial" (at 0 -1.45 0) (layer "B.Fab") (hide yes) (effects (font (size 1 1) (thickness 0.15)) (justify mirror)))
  (pad "" smd circle (at 0 0 180) (size 0.5 0.5) (layers "B.Cu" "B.Mask") (solder_mask_margin 0.25) (clearance 0.35)))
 (gr_arc (start 85 53.5) (mid 85.732233 51.732233) (end 87.5 51) (stroke (width 0.05) (type default)) (layer "Edge.Cuts"))
 (gr_arc (start 94.25 74.75) (mid 94.176777 74.926777) (end 94 75) (stroke (width 0.05) (type default)) (layer "Edge.Cuts"))
 (gr_arc (start 91.75 51) (mid 93.517767 51.732233) (end 94.25 53.5) (stroke (width 0.05) (type default)) (layer "Edge.Cuts"))
 (gr_arc (start 85.25 75) (mid 85.073223 74.926777) (end 85 74.75) (stroke (width 0.05) (type default)) (layer "Edge.Cuts"))
 (gr_line (start 94.25 74.75) (end 94.25 53.5) (stroke (width 0.05) (type default)) (layer "Edge.Cuts"))
 (gr_line (start 85.25 75) (end 89.25 75) (stroke (width 0.05) (type default)) (layer "Edge.Cuts"))
 (gr_arc (start 90 75) (mid 89.625 75.375) (end 89.25 75) (stroke (width 0.05) (type default)) (layer "Edge.Cuts"))
 (gr_line (start 94 75) (end 90 75) (stroke (width 0.05) (type default)) (layer "Edge.Cuts"))
 (gr_line (start 85 53.5) (end 85 74.75) (stroke (width 0.05) (type default)) (layer "Edge.Cuts"))
 (gr_line (start 91.75 51) (end 87.5 51) (stroke (width 0.05) (type default)) (layer "Edge.Cuts"))
 (segment (start 92.456 60.96) (end 92.964 60.452) (width 1) (layer "F.Cu") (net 7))
 (segment (start 92.964 60.452) (end 92.964 56.642) (width 1) (layer "F.Cu") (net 7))
 (via (at 92.964 56.642) (size 0.6) (drill 0.3) (layers "F.Cu" "B.Cu") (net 7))
 (segment (start 88.83 56.642) (end 88.136 55.948) (width 1) (layer "B.Cu") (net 7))
 (segment (start 88.136 55.948) (end 88.136 53.848) (width 1) (layer "B.Cu") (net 7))
 (segment (start 92.964 56.642) (end 88.83 56.642) (width 1) (layer "B.Cu") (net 7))
 (segment (start 90.106 62.294) (end 89.154 63.246) (width 1) (layer "F.Cu") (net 5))
 (segment (start 91.483 59.5495) (end 91.483 58.42) (width 1) (layer "F.Cu") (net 5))
 (segment (start 90.106 61.689) (end 90.106 62.294) (width 1) (layer "F.Cu") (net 5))
 (segment (start 90.106 61.689) (end 90.106 60.9265) (width 1) (layer "F.Cu") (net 5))
 (segment (start 90.106 60.9265) (end 91.483 59.5495) (width 1) (layer "F.Cu") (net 5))
 (segment (start 92.456 65.532) (end 92.456 64.06) (width 1) (layer "F.Cu") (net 5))
 (via (at 89.154 63.246) (size 0.6) (drill 0.3) (layers "F.Cu" "B.Cu") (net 5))
 (via (at 92.456 65.532) (size 0.6) (drill 0.3) (layers "F.Cu" "B.Cu") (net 5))
 (segment (start 89.916 64.899) (end 90.549 65.532) (width 1) (layer "B.Cu") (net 5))
 (segment (start 89.154 63.246) (end 89.154 64.137) (width 1) (layer "B.Cu") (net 5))
 (segment (start 90.549 65.532) (end 92.456 65.532) (width 1) (layer "B.Cu") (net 5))
 (segment (start 89.154 64.137) (end 89.916 64.899) (width 1) (layer "B.Cu") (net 5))
 (segment (start 86.647 61.214) (end 86.614 61.181) (width 1) (layer "F.Cu") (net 6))
 (segment (start 86.614 59.69) (end 88.138 59.69) (width 1) (layer "F.Cu") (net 6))
 (segment (start 86.614 59.69) (end 86.614 61.181) (width 1) (layer "F.Cu") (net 6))
 (segment (start 87.884 61.214) (end 86.647 61.214) (width 1) (layer "F.Cu") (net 6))
 (segment (start 88.138 59.69) (end 89.408 58.42) (width 1) (layer "F.Cu") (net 6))
 (via (at 87.884 61.214) (size 0.6) (drill 0.3) (layers "F.Cu" "B.Cu") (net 6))
 (segment (start 89.916 58.674) (end 89.916 59.182) (width 1) (layer "B.Cu") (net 6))
 (segment (start 89.916 59.182) (end 87.884 61.214) (width 1) (layer "B.Cu") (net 6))
 (segment (start 86.614 55.845) (end 88.611 53.848) (width 1) (layer "F.Cu") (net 3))
 (segment (start 86.614 56.59) (end 86.614 55.845) (width 1) (layer "F.Cu") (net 3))
 (segment (start 89.586 67.564) (end 92.456 67.564) (width 1) (layer "F.Cu") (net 2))
 (segment (start 89.5 67.65) (end 89.586 67.564) (width 1) (layer "F.Cu") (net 2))
 (via (at 92.456 67.564) (size 0.6) (drill 0.3) (layers "F.Cu" "B.Cu") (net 2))
 (segment (start 92.6 67.708) (end 92.456 67.564) (width 1) (layer "B.Cu") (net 2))
 (segment (start 92.6 71.8875) (end 92.6 67.708) (width 1) (layer "B.Cu") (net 2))
 (segment (start 86.6 71.8875) (end 86.6 68.058) (width 1) (layer "F.Cu") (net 1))
 (segment (start 86.96 67.698) (end 86.96 67.65) (width 1) (layer "F.Cu") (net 1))
 (segment (start 86.6 68.058) (end 86.96 67.698) (width 1) (layer "F.Cu") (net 1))
 (segment (start 91.186 53.848) (end 92.964 53.848) (width 1) (layer "F.Cu") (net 4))
 (via (at 92.964 53.848) (size 0.6) (drill 0.3) (layers "F.Cu" "B.Cu") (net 4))
 (segment (start 92.964 53.848) (end 90.711 53.848) (width 1) (layer "B.Cu") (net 4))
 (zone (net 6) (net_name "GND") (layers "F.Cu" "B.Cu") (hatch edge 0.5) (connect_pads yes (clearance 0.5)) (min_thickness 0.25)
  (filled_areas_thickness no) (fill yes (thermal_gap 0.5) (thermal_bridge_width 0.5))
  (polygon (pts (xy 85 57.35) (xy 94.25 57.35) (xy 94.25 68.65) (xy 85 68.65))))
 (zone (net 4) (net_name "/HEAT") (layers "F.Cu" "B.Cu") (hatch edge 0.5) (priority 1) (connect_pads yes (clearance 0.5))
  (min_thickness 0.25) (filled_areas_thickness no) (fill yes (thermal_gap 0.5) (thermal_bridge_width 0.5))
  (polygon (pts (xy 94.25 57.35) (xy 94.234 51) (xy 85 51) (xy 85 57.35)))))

